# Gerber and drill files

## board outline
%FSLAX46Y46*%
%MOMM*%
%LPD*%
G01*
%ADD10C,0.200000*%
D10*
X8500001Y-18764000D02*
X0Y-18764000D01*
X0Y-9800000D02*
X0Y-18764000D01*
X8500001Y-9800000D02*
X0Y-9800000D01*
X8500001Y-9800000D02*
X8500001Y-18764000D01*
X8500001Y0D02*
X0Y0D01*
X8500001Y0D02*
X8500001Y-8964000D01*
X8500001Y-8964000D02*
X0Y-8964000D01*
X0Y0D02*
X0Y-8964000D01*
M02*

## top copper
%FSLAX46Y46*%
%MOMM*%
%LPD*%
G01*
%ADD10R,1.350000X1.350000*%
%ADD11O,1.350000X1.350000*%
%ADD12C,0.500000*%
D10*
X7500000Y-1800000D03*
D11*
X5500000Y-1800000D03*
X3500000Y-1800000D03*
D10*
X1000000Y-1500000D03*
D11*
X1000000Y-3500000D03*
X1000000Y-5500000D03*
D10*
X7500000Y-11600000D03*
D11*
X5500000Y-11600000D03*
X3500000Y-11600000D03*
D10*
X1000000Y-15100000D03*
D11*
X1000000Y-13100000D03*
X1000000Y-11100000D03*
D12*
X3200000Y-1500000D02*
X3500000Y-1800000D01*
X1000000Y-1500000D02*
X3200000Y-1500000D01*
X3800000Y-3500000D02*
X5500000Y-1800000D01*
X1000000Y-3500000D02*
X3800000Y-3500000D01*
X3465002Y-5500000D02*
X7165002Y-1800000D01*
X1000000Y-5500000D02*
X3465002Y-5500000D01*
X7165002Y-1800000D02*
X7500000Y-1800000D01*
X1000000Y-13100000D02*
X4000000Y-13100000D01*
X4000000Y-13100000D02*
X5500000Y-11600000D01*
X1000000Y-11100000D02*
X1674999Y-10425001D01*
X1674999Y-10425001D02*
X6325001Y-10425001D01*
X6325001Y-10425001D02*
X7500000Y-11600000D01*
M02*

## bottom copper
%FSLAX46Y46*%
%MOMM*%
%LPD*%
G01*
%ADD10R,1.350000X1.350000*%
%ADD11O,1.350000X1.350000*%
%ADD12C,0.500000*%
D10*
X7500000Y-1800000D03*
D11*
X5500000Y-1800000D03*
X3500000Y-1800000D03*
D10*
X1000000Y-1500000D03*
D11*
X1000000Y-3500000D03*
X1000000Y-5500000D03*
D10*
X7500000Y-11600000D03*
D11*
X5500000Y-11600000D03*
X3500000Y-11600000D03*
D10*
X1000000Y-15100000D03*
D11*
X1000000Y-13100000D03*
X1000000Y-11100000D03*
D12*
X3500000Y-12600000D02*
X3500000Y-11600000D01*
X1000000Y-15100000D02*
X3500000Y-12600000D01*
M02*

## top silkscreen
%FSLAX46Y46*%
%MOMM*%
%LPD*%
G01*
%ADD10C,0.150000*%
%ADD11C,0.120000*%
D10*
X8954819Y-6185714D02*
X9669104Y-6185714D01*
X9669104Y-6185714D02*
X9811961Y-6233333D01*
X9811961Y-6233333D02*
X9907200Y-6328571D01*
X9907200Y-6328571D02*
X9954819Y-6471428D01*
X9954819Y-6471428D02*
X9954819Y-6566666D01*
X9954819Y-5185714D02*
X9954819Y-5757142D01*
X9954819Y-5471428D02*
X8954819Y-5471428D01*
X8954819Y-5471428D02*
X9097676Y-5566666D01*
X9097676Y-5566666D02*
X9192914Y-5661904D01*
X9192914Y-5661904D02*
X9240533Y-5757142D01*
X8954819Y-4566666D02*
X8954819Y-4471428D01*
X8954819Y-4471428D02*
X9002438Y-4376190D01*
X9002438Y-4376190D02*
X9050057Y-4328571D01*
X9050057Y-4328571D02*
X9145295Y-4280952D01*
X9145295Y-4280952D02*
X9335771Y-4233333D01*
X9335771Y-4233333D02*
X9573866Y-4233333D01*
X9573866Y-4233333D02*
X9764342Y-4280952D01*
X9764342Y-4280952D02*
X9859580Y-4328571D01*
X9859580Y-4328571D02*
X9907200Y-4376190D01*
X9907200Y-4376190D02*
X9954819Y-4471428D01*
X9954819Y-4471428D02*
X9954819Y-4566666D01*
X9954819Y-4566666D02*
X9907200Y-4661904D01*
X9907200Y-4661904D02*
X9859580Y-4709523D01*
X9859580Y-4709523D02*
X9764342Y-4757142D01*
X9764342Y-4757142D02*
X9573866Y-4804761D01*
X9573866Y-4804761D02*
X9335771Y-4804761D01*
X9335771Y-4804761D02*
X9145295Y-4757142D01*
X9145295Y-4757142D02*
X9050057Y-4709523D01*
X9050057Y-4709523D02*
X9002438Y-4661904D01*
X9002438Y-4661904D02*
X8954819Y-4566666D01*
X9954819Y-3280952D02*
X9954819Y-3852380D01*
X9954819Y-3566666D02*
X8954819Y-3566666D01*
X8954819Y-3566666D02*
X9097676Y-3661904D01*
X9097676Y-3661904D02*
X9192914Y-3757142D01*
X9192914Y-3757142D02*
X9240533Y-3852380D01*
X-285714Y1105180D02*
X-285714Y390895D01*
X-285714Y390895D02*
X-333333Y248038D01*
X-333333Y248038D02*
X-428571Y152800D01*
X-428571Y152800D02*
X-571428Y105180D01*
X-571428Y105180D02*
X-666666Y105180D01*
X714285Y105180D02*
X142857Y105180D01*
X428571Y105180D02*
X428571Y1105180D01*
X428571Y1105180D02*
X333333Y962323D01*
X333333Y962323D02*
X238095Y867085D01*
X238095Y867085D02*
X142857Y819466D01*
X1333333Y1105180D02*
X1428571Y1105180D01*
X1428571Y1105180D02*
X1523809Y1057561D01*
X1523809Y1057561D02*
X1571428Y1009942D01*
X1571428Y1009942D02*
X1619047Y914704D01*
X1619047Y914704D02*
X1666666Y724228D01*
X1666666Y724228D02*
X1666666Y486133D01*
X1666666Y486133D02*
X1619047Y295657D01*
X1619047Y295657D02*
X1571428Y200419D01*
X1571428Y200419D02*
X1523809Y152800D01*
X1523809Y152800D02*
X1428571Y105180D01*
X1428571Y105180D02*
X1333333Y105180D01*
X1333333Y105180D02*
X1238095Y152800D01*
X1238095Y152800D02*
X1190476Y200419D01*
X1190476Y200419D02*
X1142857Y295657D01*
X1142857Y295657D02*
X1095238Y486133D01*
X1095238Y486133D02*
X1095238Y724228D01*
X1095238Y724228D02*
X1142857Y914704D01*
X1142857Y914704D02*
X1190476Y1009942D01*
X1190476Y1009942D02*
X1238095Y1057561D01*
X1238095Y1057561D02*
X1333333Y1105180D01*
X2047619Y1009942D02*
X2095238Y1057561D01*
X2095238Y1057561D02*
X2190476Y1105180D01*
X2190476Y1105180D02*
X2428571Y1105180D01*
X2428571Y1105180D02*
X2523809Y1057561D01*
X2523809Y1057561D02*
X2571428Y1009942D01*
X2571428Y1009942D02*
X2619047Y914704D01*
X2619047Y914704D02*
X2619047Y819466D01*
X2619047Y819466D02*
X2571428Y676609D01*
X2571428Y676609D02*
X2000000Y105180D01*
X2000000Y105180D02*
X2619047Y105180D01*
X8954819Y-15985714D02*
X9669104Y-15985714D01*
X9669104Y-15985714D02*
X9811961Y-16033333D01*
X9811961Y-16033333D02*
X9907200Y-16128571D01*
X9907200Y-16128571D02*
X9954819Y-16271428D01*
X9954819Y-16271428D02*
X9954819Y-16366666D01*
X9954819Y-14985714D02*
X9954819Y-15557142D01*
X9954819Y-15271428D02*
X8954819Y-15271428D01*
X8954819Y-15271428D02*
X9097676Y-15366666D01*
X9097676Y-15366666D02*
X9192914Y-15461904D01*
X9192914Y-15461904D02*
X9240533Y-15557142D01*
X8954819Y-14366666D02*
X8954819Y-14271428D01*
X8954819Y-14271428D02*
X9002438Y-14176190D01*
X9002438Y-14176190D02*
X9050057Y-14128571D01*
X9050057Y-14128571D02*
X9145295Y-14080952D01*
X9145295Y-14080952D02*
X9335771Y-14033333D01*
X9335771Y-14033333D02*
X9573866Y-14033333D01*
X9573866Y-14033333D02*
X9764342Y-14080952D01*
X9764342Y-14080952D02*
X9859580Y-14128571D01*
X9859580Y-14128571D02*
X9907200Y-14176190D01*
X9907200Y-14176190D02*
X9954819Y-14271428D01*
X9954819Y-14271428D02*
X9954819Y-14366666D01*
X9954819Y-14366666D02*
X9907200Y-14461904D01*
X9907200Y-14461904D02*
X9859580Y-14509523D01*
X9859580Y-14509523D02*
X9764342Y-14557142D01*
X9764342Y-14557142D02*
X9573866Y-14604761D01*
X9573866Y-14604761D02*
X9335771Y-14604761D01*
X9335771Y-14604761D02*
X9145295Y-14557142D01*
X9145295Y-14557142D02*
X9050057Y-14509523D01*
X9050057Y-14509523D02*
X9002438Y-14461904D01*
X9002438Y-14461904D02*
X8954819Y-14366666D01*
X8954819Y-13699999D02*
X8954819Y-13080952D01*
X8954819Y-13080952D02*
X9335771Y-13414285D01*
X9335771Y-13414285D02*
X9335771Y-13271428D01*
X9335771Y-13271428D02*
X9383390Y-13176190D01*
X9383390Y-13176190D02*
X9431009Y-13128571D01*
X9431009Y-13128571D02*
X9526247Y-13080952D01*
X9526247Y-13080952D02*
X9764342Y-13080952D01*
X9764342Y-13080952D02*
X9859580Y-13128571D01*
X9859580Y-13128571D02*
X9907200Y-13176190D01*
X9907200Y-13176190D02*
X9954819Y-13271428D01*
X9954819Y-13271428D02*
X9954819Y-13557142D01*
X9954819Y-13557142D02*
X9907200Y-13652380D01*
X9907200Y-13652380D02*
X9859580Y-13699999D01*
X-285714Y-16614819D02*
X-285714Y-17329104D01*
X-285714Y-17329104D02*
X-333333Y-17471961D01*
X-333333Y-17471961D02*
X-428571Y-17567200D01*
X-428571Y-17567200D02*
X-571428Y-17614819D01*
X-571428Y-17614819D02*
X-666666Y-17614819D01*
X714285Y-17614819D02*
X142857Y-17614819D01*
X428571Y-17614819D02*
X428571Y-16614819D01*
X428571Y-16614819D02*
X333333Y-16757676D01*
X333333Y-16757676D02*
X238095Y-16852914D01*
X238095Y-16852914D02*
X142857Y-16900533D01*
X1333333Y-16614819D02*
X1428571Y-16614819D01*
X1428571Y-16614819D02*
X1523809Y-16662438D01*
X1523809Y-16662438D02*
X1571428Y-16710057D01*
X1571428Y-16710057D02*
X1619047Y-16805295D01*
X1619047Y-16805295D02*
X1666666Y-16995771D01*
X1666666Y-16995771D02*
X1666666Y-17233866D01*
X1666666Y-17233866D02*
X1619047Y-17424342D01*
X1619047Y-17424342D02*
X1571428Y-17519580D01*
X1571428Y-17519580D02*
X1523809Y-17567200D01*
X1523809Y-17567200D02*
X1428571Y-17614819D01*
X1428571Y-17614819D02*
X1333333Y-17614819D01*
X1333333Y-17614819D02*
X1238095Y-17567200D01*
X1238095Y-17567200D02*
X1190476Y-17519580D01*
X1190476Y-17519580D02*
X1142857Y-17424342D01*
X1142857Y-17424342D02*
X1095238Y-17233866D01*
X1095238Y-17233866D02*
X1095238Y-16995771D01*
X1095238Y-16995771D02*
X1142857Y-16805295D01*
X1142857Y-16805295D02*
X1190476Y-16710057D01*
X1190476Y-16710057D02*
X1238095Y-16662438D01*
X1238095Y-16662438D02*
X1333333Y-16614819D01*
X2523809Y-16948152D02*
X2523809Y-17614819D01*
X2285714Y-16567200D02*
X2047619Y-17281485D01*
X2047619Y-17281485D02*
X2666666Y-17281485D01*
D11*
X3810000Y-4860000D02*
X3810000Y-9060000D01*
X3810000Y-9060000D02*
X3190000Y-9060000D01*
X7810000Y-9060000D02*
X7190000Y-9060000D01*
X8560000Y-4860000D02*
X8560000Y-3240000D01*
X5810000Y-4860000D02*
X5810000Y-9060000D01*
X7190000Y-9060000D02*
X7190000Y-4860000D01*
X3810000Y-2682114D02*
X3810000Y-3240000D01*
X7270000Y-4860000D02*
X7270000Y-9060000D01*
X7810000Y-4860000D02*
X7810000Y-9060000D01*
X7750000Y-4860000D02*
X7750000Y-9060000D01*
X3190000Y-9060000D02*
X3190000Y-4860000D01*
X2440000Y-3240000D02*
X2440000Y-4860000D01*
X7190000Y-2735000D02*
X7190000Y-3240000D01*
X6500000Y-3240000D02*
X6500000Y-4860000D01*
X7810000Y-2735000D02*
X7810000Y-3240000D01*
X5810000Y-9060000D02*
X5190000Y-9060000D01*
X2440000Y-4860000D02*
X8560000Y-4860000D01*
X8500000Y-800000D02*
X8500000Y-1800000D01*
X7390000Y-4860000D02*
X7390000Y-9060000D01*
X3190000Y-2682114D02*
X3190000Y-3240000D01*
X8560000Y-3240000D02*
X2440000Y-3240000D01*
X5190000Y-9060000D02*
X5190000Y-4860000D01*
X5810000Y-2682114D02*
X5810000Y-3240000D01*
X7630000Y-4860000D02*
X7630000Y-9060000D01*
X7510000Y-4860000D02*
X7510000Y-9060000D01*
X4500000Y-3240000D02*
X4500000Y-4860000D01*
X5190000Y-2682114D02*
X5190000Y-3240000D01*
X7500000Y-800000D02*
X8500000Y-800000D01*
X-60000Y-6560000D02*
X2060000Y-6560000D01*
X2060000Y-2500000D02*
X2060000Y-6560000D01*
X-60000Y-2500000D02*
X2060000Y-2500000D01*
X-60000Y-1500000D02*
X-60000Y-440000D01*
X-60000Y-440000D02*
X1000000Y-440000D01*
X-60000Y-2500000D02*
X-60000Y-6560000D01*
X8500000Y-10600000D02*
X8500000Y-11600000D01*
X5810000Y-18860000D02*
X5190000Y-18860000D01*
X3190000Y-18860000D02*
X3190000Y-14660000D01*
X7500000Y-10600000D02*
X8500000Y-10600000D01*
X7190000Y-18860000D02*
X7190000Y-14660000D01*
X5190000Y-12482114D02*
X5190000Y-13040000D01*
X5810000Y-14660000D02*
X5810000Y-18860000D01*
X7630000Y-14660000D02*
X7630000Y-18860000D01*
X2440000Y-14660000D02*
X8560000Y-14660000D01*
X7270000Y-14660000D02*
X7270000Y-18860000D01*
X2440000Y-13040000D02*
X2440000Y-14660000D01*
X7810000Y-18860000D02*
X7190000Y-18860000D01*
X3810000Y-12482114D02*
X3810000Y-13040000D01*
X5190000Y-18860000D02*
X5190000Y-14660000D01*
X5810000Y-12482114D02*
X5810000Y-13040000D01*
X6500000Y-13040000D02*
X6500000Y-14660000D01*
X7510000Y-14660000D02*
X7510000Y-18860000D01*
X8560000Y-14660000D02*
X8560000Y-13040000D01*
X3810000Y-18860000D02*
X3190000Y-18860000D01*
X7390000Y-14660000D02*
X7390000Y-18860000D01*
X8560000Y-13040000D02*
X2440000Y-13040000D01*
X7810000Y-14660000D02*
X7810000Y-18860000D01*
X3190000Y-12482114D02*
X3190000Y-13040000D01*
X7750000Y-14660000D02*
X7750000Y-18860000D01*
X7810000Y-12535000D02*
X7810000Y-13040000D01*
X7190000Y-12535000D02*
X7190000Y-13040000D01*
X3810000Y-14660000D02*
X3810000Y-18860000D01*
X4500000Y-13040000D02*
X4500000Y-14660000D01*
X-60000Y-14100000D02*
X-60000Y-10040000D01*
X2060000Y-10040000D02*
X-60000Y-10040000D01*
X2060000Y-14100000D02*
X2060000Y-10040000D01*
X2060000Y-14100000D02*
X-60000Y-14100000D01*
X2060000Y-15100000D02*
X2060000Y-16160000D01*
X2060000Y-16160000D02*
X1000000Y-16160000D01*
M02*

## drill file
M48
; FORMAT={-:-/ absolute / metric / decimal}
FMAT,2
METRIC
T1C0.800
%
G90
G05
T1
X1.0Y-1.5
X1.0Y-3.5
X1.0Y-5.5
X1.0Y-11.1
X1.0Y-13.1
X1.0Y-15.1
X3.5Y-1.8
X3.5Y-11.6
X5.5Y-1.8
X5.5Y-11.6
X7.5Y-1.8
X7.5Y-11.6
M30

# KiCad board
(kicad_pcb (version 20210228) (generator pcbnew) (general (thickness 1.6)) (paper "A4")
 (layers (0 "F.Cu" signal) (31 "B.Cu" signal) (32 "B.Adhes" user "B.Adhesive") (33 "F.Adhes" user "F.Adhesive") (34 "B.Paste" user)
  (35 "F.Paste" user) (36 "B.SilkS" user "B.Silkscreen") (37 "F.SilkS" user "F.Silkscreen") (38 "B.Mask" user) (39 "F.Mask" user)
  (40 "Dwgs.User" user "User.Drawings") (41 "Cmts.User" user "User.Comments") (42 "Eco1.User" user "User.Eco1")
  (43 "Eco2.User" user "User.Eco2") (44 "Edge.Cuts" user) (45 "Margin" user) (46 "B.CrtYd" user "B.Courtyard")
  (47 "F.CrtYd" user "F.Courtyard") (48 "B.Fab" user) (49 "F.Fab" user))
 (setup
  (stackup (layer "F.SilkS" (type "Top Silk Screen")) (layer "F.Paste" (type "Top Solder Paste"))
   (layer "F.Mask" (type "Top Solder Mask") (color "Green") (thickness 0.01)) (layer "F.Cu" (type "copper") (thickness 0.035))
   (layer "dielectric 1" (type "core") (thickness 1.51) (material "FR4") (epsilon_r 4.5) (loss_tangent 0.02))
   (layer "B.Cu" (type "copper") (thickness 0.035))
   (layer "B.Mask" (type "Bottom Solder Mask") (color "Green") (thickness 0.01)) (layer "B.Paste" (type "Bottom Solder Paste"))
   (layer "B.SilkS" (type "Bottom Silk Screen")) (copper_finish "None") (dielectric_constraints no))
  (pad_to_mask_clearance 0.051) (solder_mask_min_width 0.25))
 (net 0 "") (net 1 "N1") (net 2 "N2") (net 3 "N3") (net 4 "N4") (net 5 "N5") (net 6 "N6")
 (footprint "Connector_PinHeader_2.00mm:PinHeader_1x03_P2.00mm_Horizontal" (layer "F.Cu") (at 7.5 1.8 -90)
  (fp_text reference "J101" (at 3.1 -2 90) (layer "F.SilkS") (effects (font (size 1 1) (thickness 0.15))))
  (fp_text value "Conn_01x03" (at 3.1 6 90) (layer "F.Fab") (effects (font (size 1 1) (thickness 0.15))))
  (fp_line (start 3.06 3.69) (end 7.26 3.69) (layer "F.SilkS") (width 0.12))
  (fp_line (start 7.26 3.69) (end 7.26 4.31) (layer "F.SilkS") (width 0.12))
  (fp_line (start 7.26 -0.31) (end 7.26 0.31) (layer "F.SilkS") (width 0.12))
  (fp_line (start 3.06 -1.06) (end 1.44 -1.06) (layer "F.SilkS") (width 0.12))
  (fp_line (start 3.06 1.69) (end 7.26 1.69) (layer "F.SilkS") (width 0.12))
  (fp_line (start 7.26 0.31) (end 3.06 0.31) (layer "F.SilkS") (width 0.12))
  (fp_line (start 0.882114 3.69) (end 1.44 3.69) (layer "F.SilkS") (width 0.12))
  (fp_line (start 3.06 0.23) (end 7.26 0.23) (layer "F.SilkS") (width 0.12))
  (fp_line (start 3.06 -0.31) (end 7.26 -0.31) (layer "F.SilkS") (width 0.12))
  (fp_line (start 3.06 -0.25) (end 7.26 -0.25) (layer "F.SilkS") (width 0.12))
  (fp_line (start 7.26 4.31) (end 3.06 4.31) (layer "F.SilkS") (width 0.12))
  (fp_line (start 1.44 5.06) (end 3.06 5.06) (layer "F.SilkS") (width 0.12))
  (fp_line (start 0.935 0.31) (end 1.44 0.31) (layer "F.SilkS") (width 0.12))
  (fp_line (start 1.44 1) (end 3.06 1) (layer "F.SilkS") (width 0.12))
  (fp_line (start 0.935 -0.31) (end 1.44 -0.31) (layer "F.SilkS") (width 0.12))
  (fp_line (start 7.26 1.69) (end 7.26 2.31) (layer "F.SilkS") (width 0.12))
  (fp_line (start 3.06 5.06) (end 3.06 -1.06) (layer "F.SilkS") (width 0.12))
  (fp_line (start -1 -1) (end 0 -1) (layer "F.SilkS") (width 0.12))
  (fp_line (start 3.06 0.11) (end 7.26 0.11) (layer "F.SilkS") (width 0.12))
  (fp_line (start 0.882114 4.31) (end 1.44 4.31) (layer "F.SilkS") (width 0.12))
  (fp_line (start 1.44 -1.06) (end 1.44 5.06) (layer "F.SilkS") (width 0.12))
  (fp_line (start 7.26 2.31) (end 3.06 2.31) (layer "F.SilkS") (width 0.12))
  (fp_line (start 0.882114 1.69) (end 1.44 1.69) (layer "F.SilkS") (width 0.12))
  (fp_line (start 3.06 -0.13) (end 7.26 -0.13) (layer "F.SilkS") (width 0.12))
  (fp_line (start 3.06 -0.01) (end 7.26 -0.01) (layer "F.SilkS") (width 0.12))
  (fp_line (start 1.44 3) (end 3.06 3) (layer "F.SilkS") (width 0.12))
  (fp_line (start 0.882114 2.31) (end 1.44 2.31) (layer "F.SilkS") (width 0.12))
  (fp_line (start -1 0) (end -1 -1) (layer "F.SilkS") (width 0.12))
  (pad "1" thru_hole rect (at 0 0 270) (locked) (size 1.35 1.35) (drill 0.8) (layers *.Cu *.Mask) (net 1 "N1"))
  (pad "2" thru_hole oval (at 0 2 270) (locked) (size 1.35 1.35) (drill 0.8) (layers *.Cu *.Mask) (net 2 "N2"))
  (pad "3" thru_hole oval (at 0 4 270) (locked) (size 1.35 1.35) (drill 0.8) (layers *.Cu *.Mask) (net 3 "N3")))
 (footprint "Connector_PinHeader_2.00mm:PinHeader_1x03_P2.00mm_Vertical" (layer "F.Cu") (at 1 1.5)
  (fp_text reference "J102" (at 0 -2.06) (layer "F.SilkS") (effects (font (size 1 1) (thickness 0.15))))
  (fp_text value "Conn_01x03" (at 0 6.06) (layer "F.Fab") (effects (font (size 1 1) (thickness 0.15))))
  (fp_line (start -1.06 5.06) (end 1.06 5.06) (layer "F.SilkS") (width 0.12))
  (fp_line (start 1.06 1) (end 1.06 5.06) (layer "F.SilkS") (width 0.12))
  (fp_line (start -1.06 1) (end 1.06 1) (layer "F.SilkS") (width 0.12))
  (fp_line (start -1.06 0) (end -1.06 -1.06) (layer "F.SilkS") (width 0.12))
  (fp_line (start -1.06 -1.06) (end 0 -1.06) (layer "F.SilkS") (width 0.12))
  (fp_line (start -1.06 1) (end -1.06 5.06) (layer "F.SilkS") (width 0.12))
  (pad "1" thru_hole rect (at 0 0) (locked) (size 1.35 1.35) (drill 0.8) (layers *.Cu *.Mask) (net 3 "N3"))
  (pad "2" thru_hole oval (at 0 2) (locked) (size 1.35 1.35) (drill 0.8) (layers *.Cu *.Mask) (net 2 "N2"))
  (pad "3" thru_hole oval (at 0 4) (locked) (size 1.35 1.35) (drill 0.8) (layers *.Cu *.Mask) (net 1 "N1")))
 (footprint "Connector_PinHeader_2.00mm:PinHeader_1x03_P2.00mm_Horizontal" (layer "F.Cu") (at 7.5 11.6 -90)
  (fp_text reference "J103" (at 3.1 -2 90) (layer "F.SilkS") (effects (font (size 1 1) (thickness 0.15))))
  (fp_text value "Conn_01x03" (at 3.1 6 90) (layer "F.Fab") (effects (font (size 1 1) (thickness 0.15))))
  (fp_line (start -1 -1) (end 0 -1) (layer "F.SilkS") (width 0.12))
  (fp_line (start 7.26 1.69) (end 7.26 2.31) (layer "F.SilkS") (width 0.12))
  (fp_line (start 7.26 4.31) (end 3.06 4.31) (layer "F.SilkS") (width 0.12))
  (fp_line (start -1 0) (end -1 -1) (layer "F.SilkS") (width 0.12))
  (fp_line (start 7.26 0.31) (end 3.06 0.31) (layer "F.SilkS") (width 0.12))
  (fp_line (start 0.882114 2.31) (end 1.44 2.31) (layer "F.SilkS") (width 0.12))
  (fp_line (start 3.06 1.69) (end 7.26 1.69) (layer "F.SilkS") (width 0.12))
  (fp_line (start 3.06 -0.13) (end 7.26 -0.13) (layer "F.SilkS") (width 0.12))
  (fp_line (start 3.06 5.06) (end 3.06 -1.06) (layer "F.SilkS") (width 0.12))
  (fp_line (start 3.06 0.23) (end 7.26 0.23) (layer "F.SilkS") (width 0.12))
  (fp_line (start 1.44 5.06) (end 3.06 5.06) (layer "F.SilkS") (width 0.12))
  (fp_line (start 7.26 -0.31) (end 7.26 0.31) (layer "F.SilkS") (width 0.12))
  (fp_line (start 0.882114 3.69) (end 1.44 3.69) (layer "F.SilkS") (width 0.12))
  (fp_line (start 7.26 2.31) (end 3.06 2.31) (layer "F.SilkS") (width 0.12))
  (fp_line (start 0.882114 1.69) (end 1.44 1.69) (layer "F.SilkS") (width 0.12))
  (fp_line (start 1.44 1) (end 3.06 1) (layer "F.SilkS") (width 0.12))
  (fp_line (start 3.06 -0.01) (end 7.26 -0.01) (layer "F.SilkS") (width 0.12))
  (fp_line (start 3.06 -1.06) (end 1.44 -1.06) (layer "F.SilkS") (width 0.12))
  (fp_line (start 7.26 3.69) (end 7.26 4.31) (layer "F.SilkS") (width 0.12))
  (fp_line (start 3.06 0.11) (end 7.26 0.11) (layer "F.SilkS") (width 0.12))
  (fp_line (start 1.44 -1.06) (end 1.44 5.06) (layer "F.SilkS") (width 0.12))
  (fp_line (start 3.06 -0.31) (end 7.26 -0.31) (layer "F.SilkS") (width 0.12))
  (fp_line (start 0.882114 4.31) (end 1.44 4.31) (layer "F.SilkS") (width 0.12))
  (fp_line (start 3.06 -0.25) (end 7.26 -0.25) (layer "F.SilkS") (width 0.12))
  (fp_line (start 0.935 -0.31) (end 1.44 -0.31) (layer "F.SilkS") (width 0.12))
  (fp_line (start 0.935 0.31) (end 1.44 0.31) (layer "F.SilkS") (width 0.12))
  (fp_line (start 3.06 3.69) (end 7.26 3.69) (layer "F.SilkS") (width 0.12))
  (fp_line (start 1.44 3) (end 3.06 3) (layer "F.SilkS") (width 0.12))
  (pad "1" thru_hole rect (at 0 0 270) (locked) (size 1.35 1.35) (drill 0.8) (layers *.Cu *.Mask) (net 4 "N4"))
  (pad "2" thru_hole oval (at 0 2 270) (locked) (size 1.35 1.35) (drill 0.8) (layers *.Cu *.Mask) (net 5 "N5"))
  (pad "3" thru_hole oval (at 0 4 270) (locked) (size 1.35 1.35) (drill 0.8) (layers *.Cu *.Mask) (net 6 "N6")))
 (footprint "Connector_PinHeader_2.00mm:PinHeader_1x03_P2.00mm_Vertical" (layer "F.Cu") (at 1 15.1 180)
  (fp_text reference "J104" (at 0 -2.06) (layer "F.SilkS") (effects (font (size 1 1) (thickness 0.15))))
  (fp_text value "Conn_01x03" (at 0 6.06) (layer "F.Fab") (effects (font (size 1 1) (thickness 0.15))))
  (fp_line (start 1.06 1) (end 1.06 5.06) (layer "F.SilkS") (width 0.12))
  (fp_line (start -1.06 5.06) (end 1.06 5.06) (layer "F.SilkS") (width 0.12))
  (fp_line (start -1.06 1) (end -1.06 5.06) (layer "F.SilkS") (width 0.12))
  (fp_line (start -1.06 1) (end 1.06 1) (layer "F.SilkS") (width 0.12))
  (fp_line (start -1.06 0) (end -1.06 -1.06) (layer "F.SilkS") (width 0.12))
  (fp_line (start -1.06 -1.06) (end 0 -1.06) (layer "F.SilkS") (width 0.12))
  (pad "1" thru_hole rect (at 0 0 180) (locked) (size 1.35 1.35) (drill 0.8) (layers *.Cu *.Mask) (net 6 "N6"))
  (pad "2" thru_hole oval (at 0 2 180) (locked) (size 1.35 1.35) (drill 0.8) (layers *.Cu *.Mask) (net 5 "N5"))
  (pad "3" thru_hole oval (at 0 4 180) (locked) (size 1.35 1.35) (drill 0.8) (layers *.Cu *.Mask) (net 4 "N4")))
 (gr_line (start 8.500001 18.764) (end 0 18.764) (layer "Edge.Cuts") (width 0.2))
 (gr_line (start 0 9.8) (end 0 18.764) (layer "Edge.Cuts") (width 0.2))
 (gr_line (start 8.500001 9.8) (end 0 9.8) (layer "Edge.Cuts") (width 0.2))
 (gr_line (start 8.500001 9.8) (end 8.500001 18.764) (layer "Edge.Cuts") (width 0.2))
 (gr_line (start 8.500001 0) (end 0 0) (layer "Edge.Cuts") (width 0.2))
 (gr_line (start 8.500001 0) (end 8.500001 8.964) (layer "Edge.Cuts") (width 0.2))
 (gr_line (start 8.500001 8.964) (end 0 8.964) (layer "Edge.Cuts") (width 0.2))
 (gr_line (start 0 0) (end 0 8.964) (layer "Edge.Cuts") (width 0.2))
 (segment (start 3.2 1.5) (end 3.5 1.8) (width 0.5) (layer "F.Cu") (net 3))
 (segment (start 1 1.5) (end 3.2 1.5) (width 0.5) (layer "F.Cu") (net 3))
 (segment (start 3.8 3.5) (end 5.5 1.8) (width 0.5) (layer "F.Cu") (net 2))
 (segment (start 1 3.5) (end 3.8 3.5) (width 0.5) (layer "F.Cu") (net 2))
 (segment (start 3.465002 5.5) (end 7.165002 1.8) (width 0.5) (layer "F.Cu") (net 1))
 (segment (start 1 5.5) (end 3.465002 5.5) (width 0.5) (layer "F.Cu") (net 1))
 (segment (start 7.165002 1.8) (end 7.5 1.8) (width 0.5) (layer "F.Cu") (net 1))
 (segment (start 3.5 12.6) (end 3.5 11.6) (width 0.5) (layer "B.Cu") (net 6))
 (segment (start 1 15.1) (end 3.5 12.6) (width 0.5) (layer "B.Cu") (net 6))
 (segment (start 1 13.1) (end 4 13.1) (width 0.5) (layer "F.Cu") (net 5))
 (segment (start 4 13.1) (end 5.5 11.6) (width 0.5) (layer "F.Cu") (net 5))
 (segment (start 1 11.1) (end 1.674999 10.425001) (width 0.5) (layer "F.Cu") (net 4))
 (segment (start 1.674999 10.425001) (end 6.325001 10.425001) (width 0.5) (layer "F.Cu") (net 4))
 (segment (start 6.325001 10.425001) (end 7.5 11.6) (width 0.5) (layer "F.Cu") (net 4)))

